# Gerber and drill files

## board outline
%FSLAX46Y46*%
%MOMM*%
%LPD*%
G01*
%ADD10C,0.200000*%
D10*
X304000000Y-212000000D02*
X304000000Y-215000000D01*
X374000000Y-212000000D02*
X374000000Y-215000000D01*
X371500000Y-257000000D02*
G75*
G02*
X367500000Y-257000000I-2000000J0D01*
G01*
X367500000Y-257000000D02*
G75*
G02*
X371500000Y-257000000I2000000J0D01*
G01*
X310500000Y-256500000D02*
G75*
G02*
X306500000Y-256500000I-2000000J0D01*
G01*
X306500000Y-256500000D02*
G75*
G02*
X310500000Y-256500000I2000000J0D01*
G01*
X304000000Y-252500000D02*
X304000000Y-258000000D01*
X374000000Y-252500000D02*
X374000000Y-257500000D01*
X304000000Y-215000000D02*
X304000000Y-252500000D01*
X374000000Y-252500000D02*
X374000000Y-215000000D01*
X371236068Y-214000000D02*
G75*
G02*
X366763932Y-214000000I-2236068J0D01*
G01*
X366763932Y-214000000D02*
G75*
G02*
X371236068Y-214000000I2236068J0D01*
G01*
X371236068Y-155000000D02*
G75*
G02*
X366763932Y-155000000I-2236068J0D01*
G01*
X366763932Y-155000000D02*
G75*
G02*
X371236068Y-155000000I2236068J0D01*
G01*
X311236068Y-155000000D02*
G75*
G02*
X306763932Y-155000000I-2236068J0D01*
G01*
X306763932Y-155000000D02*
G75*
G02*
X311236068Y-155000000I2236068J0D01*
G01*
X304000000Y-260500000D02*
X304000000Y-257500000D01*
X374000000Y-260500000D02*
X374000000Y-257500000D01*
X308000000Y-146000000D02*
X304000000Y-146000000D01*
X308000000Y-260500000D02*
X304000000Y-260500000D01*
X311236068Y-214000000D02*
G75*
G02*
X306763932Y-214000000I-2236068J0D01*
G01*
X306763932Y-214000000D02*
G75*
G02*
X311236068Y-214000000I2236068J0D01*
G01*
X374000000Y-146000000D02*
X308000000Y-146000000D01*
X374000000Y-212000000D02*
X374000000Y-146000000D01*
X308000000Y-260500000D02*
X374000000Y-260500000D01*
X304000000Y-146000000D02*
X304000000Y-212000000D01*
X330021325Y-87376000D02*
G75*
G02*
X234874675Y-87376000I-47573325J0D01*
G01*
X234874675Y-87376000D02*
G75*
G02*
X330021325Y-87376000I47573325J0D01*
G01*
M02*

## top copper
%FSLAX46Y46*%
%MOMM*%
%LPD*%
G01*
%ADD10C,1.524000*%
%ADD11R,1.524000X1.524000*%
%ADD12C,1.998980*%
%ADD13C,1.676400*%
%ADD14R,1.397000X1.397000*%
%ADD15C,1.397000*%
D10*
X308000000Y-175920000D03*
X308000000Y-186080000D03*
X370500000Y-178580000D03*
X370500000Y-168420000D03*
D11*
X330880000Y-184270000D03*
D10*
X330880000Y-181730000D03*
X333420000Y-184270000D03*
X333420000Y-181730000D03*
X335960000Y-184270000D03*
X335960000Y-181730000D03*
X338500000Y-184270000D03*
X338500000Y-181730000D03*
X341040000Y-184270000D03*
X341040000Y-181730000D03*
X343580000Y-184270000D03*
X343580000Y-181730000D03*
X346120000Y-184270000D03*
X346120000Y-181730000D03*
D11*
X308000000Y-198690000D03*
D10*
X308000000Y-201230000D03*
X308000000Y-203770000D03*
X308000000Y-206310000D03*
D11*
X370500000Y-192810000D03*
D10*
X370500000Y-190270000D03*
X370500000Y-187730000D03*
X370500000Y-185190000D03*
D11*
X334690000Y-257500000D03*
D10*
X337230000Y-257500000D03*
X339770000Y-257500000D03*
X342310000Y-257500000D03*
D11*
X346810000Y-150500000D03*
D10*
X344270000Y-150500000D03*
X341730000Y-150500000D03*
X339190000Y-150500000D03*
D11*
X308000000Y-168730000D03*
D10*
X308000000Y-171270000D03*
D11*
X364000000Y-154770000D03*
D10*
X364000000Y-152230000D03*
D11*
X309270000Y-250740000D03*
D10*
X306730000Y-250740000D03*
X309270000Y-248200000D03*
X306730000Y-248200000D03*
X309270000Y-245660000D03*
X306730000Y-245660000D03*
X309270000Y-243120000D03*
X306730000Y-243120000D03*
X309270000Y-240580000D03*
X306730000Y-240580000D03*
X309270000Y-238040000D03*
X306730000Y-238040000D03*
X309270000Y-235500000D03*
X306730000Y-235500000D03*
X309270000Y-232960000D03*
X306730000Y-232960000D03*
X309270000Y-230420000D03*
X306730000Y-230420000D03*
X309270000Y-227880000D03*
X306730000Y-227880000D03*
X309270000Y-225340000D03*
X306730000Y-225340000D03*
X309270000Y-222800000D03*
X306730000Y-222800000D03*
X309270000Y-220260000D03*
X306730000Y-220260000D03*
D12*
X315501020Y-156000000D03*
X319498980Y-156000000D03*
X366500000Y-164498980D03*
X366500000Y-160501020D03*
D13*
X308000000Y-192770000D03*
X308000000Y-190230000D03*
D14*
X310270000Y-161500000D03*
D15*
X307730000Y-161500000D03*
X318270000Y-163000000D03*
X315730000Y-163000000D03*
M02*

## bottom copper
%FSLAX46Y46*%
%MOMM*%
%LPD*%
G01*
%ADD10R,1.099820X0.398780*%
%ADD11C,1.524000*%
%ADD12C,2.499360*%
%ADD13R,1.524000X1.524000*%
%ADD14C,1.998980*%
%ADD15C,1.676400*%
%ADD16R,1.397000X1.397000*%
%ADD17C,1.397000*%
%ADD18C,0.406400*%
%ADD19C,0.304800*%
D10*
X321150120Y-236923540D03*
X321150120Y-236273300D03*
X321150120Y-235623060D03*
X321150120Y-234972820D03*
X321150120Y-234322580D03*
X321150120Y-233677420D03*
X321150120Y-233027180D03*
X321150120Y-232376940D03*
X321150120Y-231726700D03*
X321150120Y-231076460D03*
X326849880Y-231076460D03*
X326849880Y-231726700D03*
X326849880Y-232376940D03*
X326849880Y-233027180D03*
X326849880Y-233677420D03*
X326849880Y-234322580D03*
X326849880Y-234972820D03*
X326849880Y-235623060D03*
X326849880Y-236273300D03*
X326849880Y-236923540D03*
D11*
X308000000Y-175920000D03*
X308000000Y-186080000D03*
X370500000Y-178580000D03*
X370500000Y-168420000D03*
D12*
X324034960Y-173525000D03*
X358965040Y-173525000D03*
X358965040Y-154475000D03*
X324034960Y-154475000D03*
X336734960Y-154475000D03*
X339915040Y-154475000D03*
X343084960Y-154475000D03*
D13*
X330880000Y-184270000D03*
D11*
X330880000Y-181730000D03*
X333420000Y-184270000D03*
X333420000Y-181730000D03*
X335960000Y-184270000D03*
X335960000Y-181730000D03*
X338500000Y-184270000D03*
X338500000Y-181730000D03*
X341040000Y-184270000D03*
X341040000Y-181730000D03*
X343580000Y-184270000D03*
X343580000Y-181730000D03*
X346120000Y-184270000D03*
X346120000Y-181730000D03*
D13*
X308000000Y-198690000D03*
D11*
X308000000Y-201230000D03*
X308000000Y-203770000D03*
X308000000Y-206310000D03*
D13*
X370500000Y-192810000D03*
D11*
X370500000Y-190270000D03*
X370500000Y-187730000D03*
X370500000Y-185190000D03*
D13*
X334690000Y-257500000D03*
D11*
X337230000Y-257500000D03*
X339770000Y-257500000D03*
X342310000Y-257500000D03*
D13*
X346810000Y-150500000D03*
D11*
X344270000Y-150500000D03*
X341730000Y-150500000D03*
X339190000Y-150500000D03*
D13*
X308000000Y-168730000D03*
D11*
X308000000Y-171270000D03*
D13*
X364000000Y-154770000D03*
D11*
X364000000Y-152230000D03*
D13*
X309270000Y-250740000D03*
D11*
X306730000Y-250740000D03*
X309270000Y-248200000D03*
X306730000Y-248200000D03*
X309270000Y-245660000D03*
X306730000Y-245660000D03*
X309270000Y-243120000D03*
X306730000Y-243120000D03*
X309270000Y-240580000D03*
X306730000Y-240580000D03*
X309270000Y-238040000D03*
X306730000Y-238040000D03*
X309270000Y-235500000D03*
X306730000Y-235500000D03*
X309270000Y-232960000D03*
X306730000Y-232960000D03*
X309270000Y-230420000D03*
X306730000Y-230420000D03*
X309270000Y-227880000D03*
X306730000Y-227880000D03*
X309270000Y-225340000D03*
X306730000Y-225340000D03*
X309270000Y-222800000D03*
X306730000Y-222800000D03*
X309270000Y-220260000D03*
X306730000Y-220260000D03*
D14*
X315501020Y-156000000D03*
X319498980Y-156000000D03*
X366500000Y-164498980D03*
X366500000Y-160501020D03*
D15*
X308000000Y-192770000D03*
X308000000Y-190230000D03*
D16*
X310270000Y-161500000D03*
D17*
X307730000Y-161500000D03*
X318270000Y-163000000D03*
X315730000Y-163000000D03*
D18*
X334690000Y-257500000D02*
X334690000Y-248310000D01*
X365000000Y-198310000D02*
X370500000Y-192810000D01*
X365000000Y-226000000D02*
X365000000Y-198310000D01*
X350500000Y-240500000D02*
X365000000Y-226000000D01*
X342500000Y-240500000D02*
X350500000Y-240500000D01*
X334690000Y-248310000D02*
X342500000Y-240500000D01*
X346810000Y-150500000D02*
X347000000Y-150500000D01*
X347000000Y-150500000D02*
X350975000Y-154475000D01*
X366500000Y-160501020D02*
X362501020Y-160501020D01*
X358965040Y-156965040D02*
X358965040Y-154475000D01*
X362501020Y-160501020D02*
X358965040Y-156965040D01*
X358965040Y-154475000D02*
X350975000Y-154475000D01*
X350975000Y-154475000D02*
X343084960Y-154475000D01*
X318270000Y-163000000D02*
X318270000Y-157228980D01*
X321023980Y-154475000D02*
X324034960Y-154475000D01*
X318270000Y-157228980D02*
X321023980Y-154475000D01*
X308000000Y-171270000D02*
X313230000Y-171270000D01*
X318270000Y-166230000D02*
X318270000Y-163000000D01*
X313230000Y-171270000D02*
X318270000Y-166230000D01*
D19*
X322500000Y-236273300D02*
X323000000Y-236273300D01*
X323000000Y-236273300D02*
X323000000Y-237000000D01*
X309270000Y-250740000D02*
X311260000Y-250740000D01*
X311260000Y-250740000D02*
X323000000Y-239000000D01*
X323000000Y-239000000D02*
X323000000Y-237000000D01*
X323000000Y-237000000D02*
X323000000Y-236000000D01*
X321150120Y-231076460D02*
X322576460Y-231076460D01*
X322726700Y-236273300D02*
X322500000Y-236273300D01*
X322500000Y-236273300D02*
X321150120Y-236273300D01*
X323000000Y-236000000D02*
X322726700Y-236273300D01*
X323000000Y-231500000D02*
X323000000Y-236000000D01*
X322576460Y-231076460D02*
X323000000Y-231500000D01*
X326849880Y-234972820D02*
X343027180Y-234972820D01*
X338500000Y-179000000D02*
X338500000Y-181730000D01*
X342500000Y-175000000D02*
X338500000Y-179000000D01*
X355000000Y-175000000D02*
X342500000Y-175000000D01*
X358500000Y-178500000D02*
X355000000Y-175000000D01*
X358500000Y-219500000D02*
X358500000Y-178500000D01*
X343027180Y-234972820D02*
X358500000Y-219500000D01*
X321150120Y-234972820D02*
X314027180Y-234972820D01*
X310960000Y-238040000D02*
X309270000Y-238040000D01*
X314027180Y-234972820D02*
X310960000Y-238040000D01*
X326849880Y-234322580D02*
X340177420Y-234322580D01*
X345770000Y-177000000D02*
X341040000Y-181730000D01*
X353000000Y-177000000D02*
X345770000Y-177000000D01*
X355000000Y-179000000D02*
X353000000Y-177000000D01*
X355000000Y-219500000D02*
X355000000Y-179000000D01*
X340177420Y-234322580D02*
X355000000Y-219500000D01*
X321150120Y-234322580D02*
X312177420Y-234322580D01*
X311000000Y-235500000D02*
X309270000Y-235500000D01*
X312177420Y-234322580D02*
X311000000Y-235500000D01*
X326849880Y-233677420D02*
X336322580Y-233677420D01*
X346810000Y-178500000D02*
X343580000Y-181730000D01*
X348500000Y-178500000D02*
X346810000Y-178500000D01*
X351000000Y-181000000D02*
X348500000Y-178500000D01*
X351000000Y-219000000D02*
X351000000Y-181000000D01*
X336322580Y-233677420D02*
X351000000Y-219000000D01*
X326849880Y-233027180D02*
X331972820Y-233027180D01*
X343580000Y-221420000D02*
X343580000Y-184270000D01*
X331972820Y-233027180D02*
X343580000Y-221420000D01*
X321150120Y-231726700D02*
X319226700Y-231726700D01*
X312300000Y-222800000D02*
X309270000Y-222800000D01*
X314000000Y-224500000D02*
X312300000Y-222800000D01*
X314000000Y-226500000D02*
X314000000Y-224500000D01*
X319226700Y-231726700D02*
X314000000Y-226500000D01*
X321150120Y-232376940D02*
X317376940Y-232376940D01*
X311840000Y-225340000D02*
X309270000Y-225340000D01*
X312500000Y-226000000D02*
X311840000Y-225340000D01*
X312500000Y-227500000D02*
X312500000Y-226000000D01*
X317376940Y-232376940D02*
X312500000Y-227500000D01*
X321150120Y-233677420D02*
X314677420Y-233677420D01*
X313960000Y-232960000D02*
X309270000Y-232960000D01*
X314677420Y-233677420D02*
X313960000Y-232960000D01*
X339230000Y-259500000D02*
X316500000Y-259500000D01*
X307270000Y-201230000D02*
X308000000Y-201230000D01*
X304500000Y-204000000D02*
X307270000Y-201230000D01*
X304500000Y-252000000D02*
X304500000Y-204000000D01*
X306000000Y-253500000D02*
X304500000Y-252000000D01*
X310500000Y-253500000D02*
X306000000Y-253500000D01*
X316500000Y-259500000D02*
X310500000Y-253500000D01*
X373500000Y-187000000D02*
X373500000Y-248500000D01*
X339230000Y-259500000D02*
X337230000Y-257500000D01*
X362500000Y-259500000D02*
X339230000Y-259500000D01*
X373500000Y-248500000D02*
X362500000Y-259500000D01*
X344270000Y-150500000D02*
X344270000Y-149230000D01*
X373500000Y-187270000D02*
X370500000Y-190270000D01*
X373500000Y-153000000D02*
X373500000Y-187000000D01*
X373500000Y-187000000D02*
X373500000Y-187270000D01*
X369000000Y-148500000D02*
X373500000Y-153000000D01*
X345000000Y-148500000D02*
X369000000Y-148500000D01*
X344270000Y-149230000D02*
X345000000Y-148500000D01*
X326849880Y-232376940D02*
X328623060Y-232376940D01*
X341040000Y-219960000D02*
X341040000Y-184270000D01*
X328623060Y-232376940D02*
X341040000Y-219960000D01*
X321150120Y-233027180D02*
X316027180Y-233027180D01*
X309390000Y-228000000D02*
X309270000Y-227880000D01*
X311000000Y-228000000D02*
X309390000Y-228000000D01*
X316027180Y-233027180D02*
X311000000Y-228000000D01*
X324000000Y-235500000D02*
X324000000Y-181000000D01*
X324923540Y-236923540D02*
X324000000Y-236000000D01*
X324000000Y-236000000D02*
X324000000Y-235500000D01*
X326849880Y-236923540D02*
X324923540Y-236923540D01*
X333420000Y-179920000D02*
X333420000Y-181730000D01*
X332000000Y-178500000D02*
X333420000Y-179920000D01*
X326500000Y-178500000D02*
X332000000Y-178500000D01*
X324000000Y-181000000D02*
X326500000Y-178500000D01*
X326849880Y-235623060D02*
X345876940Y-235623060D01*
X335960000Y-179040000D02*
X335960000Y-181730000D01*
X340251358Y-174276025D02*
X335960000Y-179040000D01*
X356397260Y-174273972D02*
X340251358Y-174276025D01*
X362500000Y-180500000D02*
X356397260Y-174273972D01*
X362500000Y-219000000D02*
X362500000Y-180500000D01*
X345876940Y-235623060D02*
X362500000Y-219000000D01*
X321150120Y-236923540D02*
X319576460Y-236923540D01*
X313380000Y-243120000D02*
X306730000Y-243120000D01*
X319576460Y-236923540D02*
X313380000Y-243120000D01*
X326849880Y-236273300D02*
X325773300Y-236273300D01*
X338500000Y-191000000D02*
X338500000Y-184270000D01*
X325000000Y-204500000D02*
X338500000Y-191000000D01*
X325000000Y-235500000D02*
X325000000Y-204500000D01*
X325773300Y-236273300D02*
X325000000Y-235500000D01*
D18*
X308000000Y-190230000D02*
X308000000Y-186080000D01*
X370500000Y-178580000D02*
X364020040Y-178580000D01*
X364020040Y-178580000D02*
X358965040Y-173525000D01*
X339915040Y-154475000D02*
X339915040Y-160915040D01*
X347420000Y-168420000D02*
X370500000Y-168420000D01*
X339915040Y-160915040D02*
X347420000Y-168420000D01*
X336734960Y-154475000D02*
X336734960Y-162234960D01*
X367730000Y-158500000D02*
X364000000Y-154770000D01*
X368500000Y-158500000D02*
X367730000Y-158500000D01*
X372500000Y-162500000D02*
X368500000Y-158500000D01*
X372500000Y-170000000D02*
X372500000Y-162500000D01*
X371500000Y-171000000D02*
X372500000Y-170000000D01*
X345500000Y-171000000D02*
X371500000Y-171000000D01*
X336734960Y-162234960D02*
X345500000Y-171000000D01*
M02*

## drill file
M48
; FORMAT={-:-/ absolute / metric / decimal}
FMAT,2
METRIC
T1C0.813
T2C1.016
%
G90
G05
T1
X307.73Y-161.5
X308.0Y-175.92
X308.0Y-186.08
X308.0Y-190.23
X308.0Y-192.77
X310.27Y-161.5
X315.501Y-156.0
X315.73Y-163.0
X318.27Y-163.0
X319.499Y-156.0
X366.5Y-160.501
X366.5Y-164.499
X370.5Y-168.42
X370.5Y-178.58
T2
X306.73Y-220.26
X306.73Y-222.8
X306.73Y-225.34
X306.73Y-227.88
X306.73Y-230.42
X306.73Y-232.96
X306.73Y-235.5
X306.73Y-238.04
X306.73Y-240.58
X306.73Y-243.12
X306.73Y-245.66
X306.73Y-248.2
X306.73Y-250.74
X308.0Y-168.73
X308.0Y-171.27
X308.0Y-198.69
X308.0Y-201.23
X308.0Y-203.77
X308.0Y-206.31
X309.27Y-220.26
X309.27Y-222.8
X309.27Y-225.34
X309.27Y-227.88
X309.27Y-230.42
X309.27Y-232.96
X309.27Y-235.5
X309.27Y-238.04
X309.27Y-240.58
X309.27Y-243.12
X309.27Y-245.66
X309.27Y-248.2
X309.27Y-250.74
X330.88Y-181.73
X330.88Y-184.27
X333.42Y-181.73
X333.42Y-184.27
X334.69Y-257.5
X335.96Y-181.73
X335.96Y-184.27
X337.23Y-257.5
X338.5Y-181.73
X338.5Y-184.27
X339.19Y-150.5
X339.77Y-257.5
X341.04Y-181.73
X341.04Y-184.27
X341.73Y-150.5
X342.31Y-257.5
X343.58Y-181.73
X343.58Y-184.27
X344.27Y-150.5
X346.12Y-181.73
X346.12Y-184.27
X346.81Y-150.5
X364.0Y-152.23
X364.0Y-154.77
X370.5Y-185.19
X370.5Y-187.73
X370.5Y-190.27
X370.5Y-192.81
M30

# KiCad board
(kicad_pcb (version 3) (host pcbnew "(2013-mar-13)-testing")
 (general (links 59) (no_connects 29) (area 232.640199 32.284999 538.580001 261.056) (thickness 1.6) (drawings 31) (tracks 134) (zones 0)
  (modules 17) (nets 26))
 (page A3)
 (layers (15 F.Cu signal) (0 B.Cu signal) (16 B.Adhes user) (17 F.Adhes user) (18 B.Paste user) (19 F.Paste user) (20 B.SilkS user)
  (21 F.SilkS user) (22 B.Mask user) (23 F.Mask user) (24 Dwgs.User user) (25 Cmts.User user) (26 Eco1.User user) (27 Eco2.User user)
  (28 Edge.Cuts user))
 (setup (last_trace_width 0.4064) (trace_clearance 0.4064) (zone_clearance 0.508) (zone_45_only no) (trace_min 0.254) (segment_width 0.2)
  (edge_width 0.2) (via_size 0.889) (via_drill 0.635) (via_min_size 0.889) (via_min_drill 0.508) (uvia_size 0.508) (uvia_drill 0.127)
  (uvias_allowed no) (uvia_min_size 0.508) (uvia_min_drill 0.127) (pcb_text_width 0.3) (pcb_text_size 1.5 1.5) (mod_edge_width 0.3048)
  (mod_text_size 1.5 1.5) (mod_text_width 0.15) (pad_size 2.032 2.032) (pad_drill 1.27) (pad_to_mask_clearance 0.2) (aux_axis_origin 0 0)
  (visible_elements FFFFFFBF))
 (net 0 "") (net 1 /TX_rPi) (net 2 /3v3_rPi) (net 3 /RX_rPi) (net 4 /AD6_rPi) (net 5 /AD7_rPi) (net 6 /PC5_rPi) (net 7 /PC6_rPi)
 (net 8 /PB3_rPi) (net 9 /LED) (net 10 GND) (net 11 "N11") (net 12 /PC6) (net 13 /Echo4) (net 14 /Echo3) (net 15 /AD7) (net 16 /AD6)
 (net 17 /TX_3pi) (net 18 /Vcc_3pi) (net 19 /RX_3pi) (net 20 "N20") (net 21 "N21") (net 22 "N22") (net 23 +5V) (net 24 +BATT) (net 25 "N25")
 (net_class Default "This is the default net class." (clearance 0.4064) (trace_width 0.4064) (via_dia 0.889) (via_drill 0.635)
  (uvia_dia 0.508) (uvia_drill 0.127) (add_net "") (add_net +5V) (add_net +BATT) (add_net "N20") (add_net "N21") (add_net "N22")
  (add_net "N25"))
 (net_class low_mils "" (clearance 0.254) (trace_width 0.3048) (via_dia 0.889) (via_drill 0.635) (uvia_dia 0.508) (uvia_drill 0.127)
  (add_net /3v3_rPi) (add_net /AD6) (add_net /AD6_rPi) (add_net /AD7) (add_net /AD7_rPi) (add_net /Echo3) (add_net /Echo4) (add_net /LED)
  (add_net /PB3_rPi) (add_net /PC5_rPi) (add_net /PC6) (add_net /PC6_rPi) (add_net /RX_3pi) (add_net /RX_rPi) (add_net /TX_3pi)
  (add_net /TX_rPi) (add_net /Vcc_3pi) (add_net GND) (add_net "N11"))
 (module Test (layer B.Cu) (at 324 234 90)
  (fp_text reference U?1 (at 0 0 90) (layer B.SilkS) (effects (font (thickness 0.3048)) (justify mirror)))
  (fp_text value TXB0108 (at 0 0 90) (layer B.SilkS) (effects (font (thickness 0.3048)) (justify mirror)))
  (pad 1 smd rect (at -2.92354 -2.84988 270) (size 0.39878 1.09982) (layers B.Cu B.Paste B.Mask) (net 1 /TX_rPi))
  (pad 2 smd rect (at -2.2733 -2.84988 270) (size 0.39878 1.09982) (layers B.Cu B.Paste B.Mask) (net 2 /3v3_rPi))
  (pad 3 smd rect (at -1.62306 -2.84988 270) (size 0.39878 1.09982) (layers B.Cu B.Paste B.Mask) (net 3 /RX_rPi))
  (pad 4 smd rect (at -0.97282 -2.84988 270) (size 0.39878 1.09982) (layers B.Cu B.Paste B.Mask) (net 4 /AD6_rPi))
  (pad 5 smd rect (at -0.32258 -2.84988 270) (size 0.39878 1.09982) (layers B.Cu B.Paste B.Mask) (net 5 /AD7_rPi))
  (pad 6 smd rect (at 0.32258 -2.84988 270) (size 0.39878 1.09982) (layers B.Cu B.Paste B.Mask) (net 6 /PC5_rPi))
  (pad 7 smd rect (at 0.97282 -2.84988 270) (size 0.39878 1.09982) (layers B.Cu B.Paste B.Mask) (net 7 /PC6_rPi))
  (pad 8 smd rect (at 1.62306 -2.84988 270) (size 0.39878 1.09982) (layers B.Cu B.Paste B.Mask) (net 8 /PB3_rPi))
  (pad 9 smd rect (at 2.2733 -2.84988 270) (size 0.39878 1.09982) (layers B.Cu B.Paste B.Mask) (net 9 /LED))
  (pad 10 smd rect (at 2.92354 -2.84988 270) (size 0.39878 1.09982) (layers B.Cu B.Paste B.Mask) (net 2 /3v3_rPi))
  (pad 11 smd rect (at 2.92354 2.84988 90) (size 0.39878 1.09982) (layers B.Cu B.Paste B.Mask) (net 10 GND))
  (pad 12 smd rect (at 2.2733 2.84988 90) (size 0.39878 1.09982) (layers B.Cu B.Paste B.Mask) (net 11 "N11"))
  (pad 13 smd rect (at 1.62306 2.84988 90) (size 0.39878 1.09982) (layers B.Cu B.Paste B.Mask) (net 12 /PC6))
  (pad 14 smd rect (at 0.97282 2.84988 90) (size 0.39878 1.09982) (layers B.Cu B.Paste B.Mask) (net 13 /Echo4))
  (pad 15 smd rect (at 0.32258 2.84988 90) (size 0.39878 1.09982) (layers B.Cu B.Paste B.Mask) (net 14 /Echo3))
  (pad 16 smd rect (at -0.32258 2.84988 90) (size 0.39878 1.09982) (layers B.Cu B.Paste B.Mask) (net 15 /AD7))
  (pad 17 smd rect (at -0.97282 2.84988 90) (size 0.39878 1.09982) (layers B.Cu B.Paste B.Mask) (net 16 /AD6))
  (pad 18 smd rect (at -1.62306 2.84988 90) (size 0.39878 1.09982) (layers B.Cu B.Paste B.Mask) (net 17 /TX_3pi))
  (pad 19 smd rect (at -2.2733 2.84988 90) (size 0.39878 1.09982) (layers B.Cu B.Paste B.Mask) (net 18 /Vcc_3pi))
  (pad 20 smd rect (at -2.92354 2.84988 90) (size 0.39878 1.09982) (layers B.Cu B.Paste B.Mask) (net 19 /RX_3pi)))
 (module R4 (layer F.Cu) (at 308 181 270) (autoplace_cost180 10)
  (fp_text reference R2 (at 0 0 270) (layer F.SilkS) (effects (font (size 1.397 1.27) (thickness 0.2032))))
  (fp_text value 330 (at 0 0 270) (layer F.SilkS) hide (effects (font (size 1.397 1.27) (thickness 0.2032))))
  (pad 1 thru_hole circle (at -5.08 0 270) (size 1.524 1.524) (drill 0.8128) (layers *.Cu *.Mask F.SilkS) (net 10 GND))
  (pad 2 thru_hole circle (at 5.08 0 270) (size 1.524 1.524) (drill 0.8128) (layers *.Cu *.Mask F.SilkS) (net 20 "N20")))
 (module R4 (layer F.Cu) (at 370.5 173.5 90) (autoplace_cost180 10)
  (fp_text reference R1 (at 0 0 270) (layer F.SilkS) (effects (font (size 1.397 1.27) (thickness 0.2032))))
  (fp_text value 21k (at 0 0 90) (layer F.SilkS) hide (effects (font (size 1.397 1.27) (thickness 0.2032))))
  (pad 1 thru_hole circle (at -5.08 0 90) (size 1.524 1.524) (drill 0.8128) (layers *.Cu *.Mask F.SilkS) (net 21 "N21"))
  (pad 2 thru_hole circle (at 5.08 0 90) (size 1.524 1.524) (drill 0.8128) (layers *.Cu *.Mask F.SilkS) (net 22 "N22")))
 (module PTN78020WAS (layer B.Cu) (at 341.5 164)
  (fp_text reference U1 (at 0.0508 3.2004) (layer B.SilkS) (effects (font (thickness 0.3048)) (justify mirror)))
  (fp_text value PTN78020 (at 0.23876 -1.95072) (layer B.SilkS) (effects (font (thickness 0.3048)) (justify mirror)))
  (pad 1 smd circle (at -17.46504 9.525) (size 2.49936 2.49936) (layers B.Cu B.Paste B.Mask) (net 10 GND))
  (pad 7 smd circle (at 17.46504 9.525) (size 2.49936 2.49936) (layers B.Cu B.Paste B.Mask) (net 21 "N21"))
  (pad 6 smd circle (at 17.46504 -9.525) (size 2.49936 2.49936) (layers B.Cu B.Paste B.Mask) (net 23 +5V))
  (pad 2 smd circle (at -17.46504 -9.525) (size 2.49936 2.49936) (layers B.Cu B.Paste B.Mask) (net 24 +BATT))
  (pad 3 smd circle (at -4.76504 -9.525) (size 2.49936 2.49936) (layers B.Cu B.Paste B.Mask) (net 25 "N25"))
  (pad 4 smd circle (at -1.58496 -9.525) (size 2.49936 2.49936) (layers B.Cu B.Paste B.Mask) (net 22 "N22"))
  (pad 5 smd circle (at 1.58496 -9.525) (size 2.49936 2.49936) (layers B.Cu B.Paste B.Mask) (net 23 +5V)))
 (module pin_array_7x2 (layer F.Cu) (at 338.5 183)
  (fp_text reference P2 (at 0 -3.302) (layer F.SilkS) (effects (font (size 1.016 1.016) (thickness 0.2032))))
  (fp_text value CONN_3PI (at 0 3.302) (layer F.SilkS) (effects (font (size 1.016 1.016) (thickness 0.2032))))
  (pad 1 thru_hole rect (at -7.62 1.27) (size 1.524 1.524) (drill 1.016) (layers *.Cu *.Mask F.SilkS) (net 10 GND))
  (pad 2 thru_hole circle (at -7.62 -1.27) (size 1.524 1.524) (drill 1.016) (layers *.Cu *.Mask F.SilkS) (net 10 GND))
  (pad 3 thru_hole circle (at -5.08 1.27) (size 1.524 1.524) (drill 1.016) (layers *.Cu *.Mask F.SilkS))
  (pad 4 thru_hole circle (at -5.08 -1.27) (size 1.524 1.524) (drill 1.016) (layers *.Cu *.Mask F.SilkS) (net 19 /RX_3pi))
  (pad 5 thru_hole circle (at -2.54 1.27) (size 1.524 1.524) (drill 1.016) (layers *.Cu *.Mask F.SilkS))
  (pad 6 thru_hole circle (at -2.54 -1.27) (size 1.524 1.524) (drill 1.016) (layers *.Cu *.Mask F.SilkS) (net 17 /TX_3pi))
  (pad 7 thru_hole circle (at 0 1.27) (size 1.524 1.524) (drill 1.016) (layers *.Cu *.Mask F.SilkS) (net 18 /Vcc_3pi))
  (pad 8 thru_hole circle (at 0 -1.27) (size 1.524 1.524) (drill 1.016) (layers *.Cu *.Mask F.SilkS) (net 16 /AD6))
  (pad 9 thru_hole circle (at 2.54 1.27) (size 1.524 1.524) (drill 1.016) (layers *.Cu *.Mask F.SilkS) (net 12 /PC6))
  (pad 10 thru_hole circle (at 2.54 -1.27) (size 1.524 1.524) (drill 1.016) (layers *.Cu *.Mask F.SilkS) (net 15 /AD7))
  (pad 11 thru_hole circle (at 5.08 1.27) (size 1.524 1.524) (drill 1.016) (layers *.Cu *.Mask F.SilkS) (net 13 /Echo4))
  (pad 12 thru_hole circle (at 5.08 -1.27) (size 1.524 1.524) (drill 1.016) (layers *.Cu *.Mask F.SilkS) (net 14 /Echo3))
  (pad 13 thru_hole circle (at 7.62 1.27) (size 1.524 1.524) (drill 1.016) (layers *.Cu *.Mask F.SilkS) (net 10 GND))
  (pad 14 thru_hole circle (at 7.62 -1.27) (size 1.524 1.524) (drill 1.016) (layers *.Cu *.Mask F.SilkS) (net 10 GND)))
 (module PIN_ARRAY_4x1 (layer F.Cu) (at 308 202.5 270)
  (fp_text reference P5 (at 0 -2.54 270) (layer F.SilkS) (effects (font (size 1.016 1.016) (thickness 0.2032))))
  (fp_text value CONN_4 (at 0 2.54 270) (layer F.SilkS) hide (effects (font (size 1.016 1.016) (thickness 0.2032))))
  (pad 1 thru_hole rect (at -3.81 0 270) (size 1.524 1.524) (drill 1.016) (layers *.Cu *.Mask F.SilkS) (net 23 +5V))
  (pad 2 thru_hole circle (at -1.27 0 270) (size 1.524 1.524) (drill 1.016) (layers *.Cu *.Mask F.SilkS) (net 12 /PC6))
  (pad 3 thru_hole circle (at 1.27 0 270) (size 1.524 1.524) (drill 1.016) (layers *.Cu *.Mask F.SilkS) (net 16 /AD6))
  (pad 4 thru_hole circle (at 3.81 0 270) (size 1.524 1.524) (drill 1.016) (layers *.Cu *.Mask F.SilkS) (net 10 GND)))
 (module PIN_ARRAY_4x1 (layer F.Cu) (at 370.5 189 90)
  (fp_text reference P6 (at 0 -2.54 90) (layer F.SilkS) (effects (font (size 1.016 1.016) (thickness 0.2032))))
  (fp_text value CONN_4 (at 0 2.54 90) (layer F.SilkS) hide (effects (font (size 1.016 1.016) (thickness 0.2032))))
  (pad 1 thru_hole rect (at -3.81 0 90) (size 1.524 1.524) (drill 1.016) (layers *.Cu *.Mask F.SilkS) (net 23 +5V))
  (pad 2 thru_hole circle (at -1.27 0 90) (size 1.524 1.524) (drill 1.016) (layers *.Cu *.Mask F.SilkS) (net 12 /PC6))
  (pad 3 thru_hole circle (at 1.27 0 90) (size 1.524 1.524) (drill 1.016) (layers *.Cu *.Mask F.SilkS) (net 15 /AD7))
  (pad 4 thru_hole circle (at 3.81 0 90) (size 1.524 1.524) (drill 1.016) (layers *.Cu *.Mask F.SilkS) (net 10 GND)))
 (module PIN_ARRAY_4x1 (layer F.Cu) (at 338.5 257.5)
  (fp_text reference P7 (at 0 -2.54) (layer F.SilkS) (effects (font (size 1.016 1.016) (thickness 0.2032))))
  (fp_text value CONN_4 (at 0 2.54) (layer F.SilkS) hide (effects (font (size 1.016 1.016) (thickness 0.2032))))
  (pad 1 thru_hole rect (at -3.81 0) (size 1.524 1.524) (drill 1.016) (layers *.Cu *.Mask F.SilkS) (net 23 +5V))
  (pad 2 thru_hole circle (at -1.27 0) (size 1.524 1.524) (drill 1.016) (layers *.Cu *.Mask F.SilkS) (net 12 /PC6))
  (pad 3 thru_hole circle (at 1.27 0) (size 1.524 1.524) (drill 1.016) (layers *.Cu *.Mask F.SilkS) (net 14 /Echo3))
  (pad 4 thru_hole circle (at 3.81 0) (size 1.524 1.524) (drill 1.016) (layers *.Cu *.Mask F.SilkS) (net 10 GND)))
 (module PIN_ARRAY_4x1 (layer F.Cu) (at 343 150.5 180)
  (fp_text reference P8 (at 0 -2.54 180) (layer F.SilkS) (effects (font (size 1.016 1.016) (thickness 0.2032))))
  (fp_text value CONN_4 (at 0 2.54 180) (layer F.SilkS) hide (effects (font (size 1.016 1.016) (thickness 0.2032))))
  (pad 1 thru_hole rect (at -3.81 0 180) (size 1.524 1.524) (drill 1.016) (layers *.Cu *.Mask F.SilkS) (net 23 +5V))
  (pad 2 thru_hole circle (at -1.27 0 180) (size 1.524 1.524) (drill 1.016) (layers *.Cu *.Mask F.SilkS) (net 12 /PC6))
  (pad 3 thru_hole circle (at 1.27 0 180) (size 1.524 1.524) (drill 1.016) (layers *.Cu *.Mask F.SilkS) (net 13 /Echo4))
  (pad 4 thru_hole circle (at 3.81 0 180) (size 1.524 1.524) (drill 1.016) (layers *.Cu *.Mask F.SilkS) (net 10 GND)))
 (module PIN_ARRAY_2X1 (layer F.Cu) (at 308 170 270)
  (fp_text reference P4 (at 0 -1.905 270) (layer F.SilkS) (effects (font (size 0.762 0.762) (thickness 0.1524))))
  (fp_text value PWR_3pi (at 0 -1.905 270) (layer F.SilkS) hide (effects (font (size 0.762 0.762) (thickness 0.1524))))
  (pad 1 thru_hole rect (at -1.27 0 270) (size 1.524 1.524) (drill 1.016) (layers *.Cu *.Mask F.SilkS) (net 10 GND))
  (pad 2 thru_hole circle (at 1.27 0 270) (size 1.524 1.524) (drill 1.016) (layers *.Cu *.Mask F.SilkS) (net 24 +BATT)))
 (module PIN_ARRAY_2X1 (layer F.Cu) (at 364 153.5 90)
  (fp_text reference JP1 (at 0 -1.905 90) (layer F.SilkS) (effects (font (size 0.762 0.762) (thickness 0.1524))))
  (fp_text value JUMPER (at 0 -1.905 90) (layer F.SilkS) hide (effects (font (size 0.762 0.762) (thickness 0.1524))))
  (pad 1 thru_hole rect (at -1.27 0 90) (size 1.524 1.524) (drill 1.016) (layers *.Cu *.Mask F.SilkS) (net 25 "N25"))
  (pad 2 thru_hole circle (at 1.27 0 90) (size 1.524 1.524) (drill 1.016) (layers *.Cu *.Mask F.SilkS) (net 10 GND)))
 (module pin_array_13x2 (layer F.Cu) (at 308 235.5 90)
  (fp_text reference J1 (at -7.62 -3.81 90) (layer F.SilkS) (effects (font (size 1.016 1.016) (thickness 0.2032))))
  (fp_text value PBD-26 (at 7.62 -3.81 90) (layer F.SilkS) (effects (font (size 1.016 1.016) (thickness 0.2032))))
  (pad 1 thru_hole rect (at -15.24 1.27 90) (size 1.524 1.524) (drill 1.016) (layers *.Cu *.Mask F.SilkS) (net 2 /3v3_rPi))
  (pad 2 thru_hole circle (at -15.24 -1.27 90) (size 1.524 1.524) (drill 1.016) (layers *.Cu *.Mask F.SilkS))
  (pad 3 thru_hole circle (at -12.7 1.27 90) (size 1.524 1.524) (drill 1.016) (layers *.Cu *.Mask F.SilkS))
  (pad 4 thru_hole circle (at -12.7 -1.27 90) (size 1.524 1.524) (drill 1.016) (layers *.Cu *.Mask F.SilkS))
  (pad 5 thru_hole circle (at -10.16 1.27 90) (size 1.524 1.524) (drill 1.016) (layers *.Cu *.Mask F.SilkS))
  (pad 6 thru_hole circle (at -10.16 -1.27 90) (size 1.524 1.524) (drill 1.016) (layers *.Cu *.Mask F.SilkS) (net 10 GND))
  (pad 7 thru_hole circle (at -7.62 1.27 90) (size 1.524 1.524) (drill 1.016) (layers *.Cu *.Mask F.SilkS) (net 1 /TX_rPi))
  (pad 8 thru_hole circle (at -7.62 -1.27 90) (size 1.524 1.524) (drill 1.016) (layers *.Cu *.Mask F.SilkS) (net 1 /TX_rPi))
  (pad 9 thru_hole circle (at -5.08 1.27 90) (size 1.524 1.524) (drill 1.016) (layers *.Cu *.Mask F.SilkS))
  (pad 10 thru_hole circle (at -5.08 -1.27 90) (size 1.524 1.524) (drill 1.016) (layers *.Cu *.Mask F.SilkS) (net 3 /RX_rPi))
  (pad 11 thru_hole circle (at -2.54 1.27 90) (size 1.524 1.524) (drill 1.016) (layers *.Cu *.Mask F.SilkS) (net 4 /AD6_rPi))
  (pad 12 thru_hole circle (at -2.54 -1.27 90) (size 1.524 1.524) (drill 1.016) (layers *.Cu *.Mask F.SilkS))
  (pad 13 thru_hole circle (at 0 1.27 90) (size 1.524 1.524) (drill 1.016) (layers *.Cu *.Mask F.SilkS) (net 5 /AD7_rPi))
  (pad 14 thru_hole circle (at 0 -1.27 90) (size 1.524 1.524) (drill 1.016) (layers *.Cu *.Mask F.SilkS))
  (pad 15 thru_hole circle (at 2.54 1.27 90) (size 1.524 1.524) (drill 1.016) (layers *.Cu *.Mask F.SilkS) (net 6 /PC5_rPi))
  (pad 16 thru_hole circle (at 2.54 -1.27 90) (size 1.524 1.524) (drill 1.016) (layers *.Cu *.Mask F.SilkS))
  (pad 17 thru_hole circle (at 5.08 1.27 90) (size 1.524 1.524) (drill 1.016) (layers *.Cu *.Mask F.SilkS))
  (pad 18 thru_hole circle (at 5.08 -1.27 90) (size 1.524 1.524) (drill 1.016) (layers *.Cu *.Mask F.SilkS))
  (pad 19 thru_hole circle (at 7.62 1.27 90) (size 1.524 1.524) (drill 1.016) (layers *.Cu *.Mask F.SilkS) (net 7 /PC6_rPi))
  (pad 20 thru_hole circle (at 7.62 -1.27 90) (size 1.524 1.524) (drill 1.016) (layers *.Cu *.Mask F.SilkS))
  (pad 21 thru_hole circle (at 10.16 1.27 90) (size 1.524 1.524) (drill 1.016) (layers *.Cu *.Mask F.SilkS) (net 8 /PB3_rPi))
  (pad 22 thru_hole circle (at 10.16 -1.27 90) (size 1.524 1.524) (drill 1.016) (layers *.Cu *.Mask F.SilkS))
  (pad 23 thru_hole circle (at 12.7 1.27 90) (size 1.524 1.524) (drill 1.016) (layers *.Cu *.Mask F.SilkS) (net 9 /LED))
  (pad 24 thru_hole circle (at 12.7 -1.27 90) (size 1.524 1.524) (drill 1.016) (layers *.Cu *.Mask F.SilkS))
  (pad 25 thru_hole circle (at 15.24 1.27 90) (size 1.524 1.524) (drill 1.016) (layers *.Cu *.Mask F.SilkS))
  (pad 26 thru_hole circle (at 15.24 -1.27 90) (size 1.524 1.524) (drill 1.016) (layers *.Cu *.Mask F.SilkS)))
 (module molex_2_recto (layer F.Cu) (at 317.5 156 180)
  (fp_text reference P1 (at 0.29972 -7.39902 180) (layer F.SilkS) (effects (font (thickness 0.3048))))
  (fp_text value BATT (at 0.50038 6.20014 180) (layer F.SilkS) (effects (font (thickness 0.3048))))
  (pad 1 thru_hole circle (at 1.99898 0 180) (size 1.99898 1.99898) (drill 0.8128) (layers *.Cu *.Mask F.SilkS) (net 10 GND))
  (pad 2 thru_hole circle (at -1.99898 0 180) (size 1.99898 1.99898) (drill 0.8128) (layers *.Cu *.Mask F.SilkS) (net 24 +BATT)))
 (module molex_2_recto (layer F.Cu) (at 366.5 162.5 270)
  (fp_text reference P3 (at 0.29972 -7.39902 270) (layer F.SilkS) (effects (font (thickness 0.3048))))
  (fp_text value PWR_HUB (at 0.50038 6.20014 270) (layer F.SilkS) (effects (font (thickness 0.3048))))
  (pad 1 thru_hole circle (at 1.99898 0 270) (size 1.99898 1.99898) (drill 0.8128) (layers *.Cu *.Mask F.SilkS) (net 10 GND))
  (pad 2 thru_hole circle (at -1.99898 0 270) (size 1.99898 1.99898) (drill 0.8128) (layers *.Cu *.Mask F.SilkS) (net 23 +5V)))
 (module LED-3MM (layer F.Cu) (at 308 191.5 90)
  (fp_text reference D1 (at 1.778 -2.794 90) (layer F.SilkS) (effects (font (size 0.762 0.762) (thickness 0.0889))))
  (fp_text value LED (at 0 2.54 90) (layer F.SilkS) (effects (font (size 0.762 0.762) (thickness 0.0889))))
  (pad 1 thru_hole circle (at -1.27 0 90) (size 1.6764 1.6764) (drill 0.8128) (layers *.Cu *.Mask F.SilkS) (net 11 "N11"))
  (pad 2 thru_hole circle (at 1.27 0 90) (size 1.6764 1.6764) (drill 0.8128) (layers *.Cu *.Mask F.SilkS) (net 20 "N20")))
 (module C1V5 (layer F.Cu) (at 309 161.5 180)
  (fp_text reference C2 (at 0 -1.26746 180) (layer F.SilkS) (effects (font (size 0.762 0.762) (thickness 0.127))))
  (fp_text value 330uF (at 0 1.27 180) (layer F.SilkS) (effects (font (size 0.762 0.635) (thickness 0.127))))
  (pad 1 thru_hole rect (at -1.27 0 180) (size 1.397 1.397) (drill 0.8128) (layers *.Cu *.Mask F.SilkS) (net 23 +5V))
  (pad 2 thru_hole circle (at 1.27 0 180) (size 1.397 1.397) (drill 0.8128) (layers *.Cu *.Mask F.SilkS) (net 10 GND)))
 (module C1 (layer F.Cu) (at 317 163 180)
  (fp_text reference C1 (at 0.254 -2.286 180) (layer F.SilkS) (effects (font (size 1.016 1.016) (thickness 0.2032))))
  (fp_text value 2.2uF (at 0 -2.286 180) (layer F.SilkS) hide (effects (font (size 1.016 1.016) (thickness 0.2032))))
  (pad 1 thru_hole circle (at -1.27 0 180) (size 1.397 1.397) (drill 0.8128) (layers *.Cu *.Mask F.SilkS) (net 24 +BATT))
  (pad 2 thru_hole circle (at 1.27 0 180) (size 1.397 1.397) (drill 0.8128) (layers *.Cu *.Mask F.SilkS) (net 10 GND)))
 (gr_line (start 304 212) (end 304 215) (angle 90) (layer Edge.Cuts) (width 0.2))
 (gr_line (start 374 212) (end 374 215) (angle 90) (layer Edge.Cuts) (width 0.2))
 (gr_circle (center 369.5 257) (end 369.5 259) (layer Edge.Cuts) (width 0.2))
 (gr_circle (center 308.5 256.5) (end 308.5 258.5) (layer Edge.Cuts) (width 0.2))
 (gr_line (start 304 252.5) (end 304 258) (angle 90) (layer Edge.Cuts) (width 0.2))
 (gr_line (start 374 252.5) (end 374 257.5) (angle 90) (layer Edge.Cuts) (width 0.2))
 (gr_line (start 304 215) (end 304 252.5) (angle 90) (layer Edge.Cuts) (width 0.2))
 (gr_line (start 374 252.5) (end 374 215) (angle 90) (layer Edge.Cuts) (width 0.2))
 (gr_circle (center 369 214) (end 370 216) (layer Edge.Cuts) (width 0.2))
 (gr_circle (center 369 155) (end 367 156) (layer Edge.Cuts) (width 0.2))
 (gr_circle (center 309 155) (end 311 156) (layer Edge.Cuts) (width 0.2))
 (gr_line (start 304 260.5) (end 304 257.5) (angle 90) (layer Edge.Cuts) (width 0.2))
 (gr_line (start 374 260.5) (end 374 257.5) (angle 90) (layer Edge.Cuts) (width 0.2))
 (gr_line (start 308 146) (end 304 146) (angle 90) (layer Edge.Cuts) (width 0.2))
 (gr_line (start 308 260.5) (end 304 260.5) (angle 90) (layer Edge.Cuts) (width 0.2))
 (gr_circle (center 309 214) (end 311 215) (layer Edge.Cuts) (width 0.2))
 (gr_line (start 374 146) (end 308 146) (angle 90) (layer Edge.Cuts) (width 0.2))
 (gr_line (start 374 212) (end 374 146) (angle 90) (layer Edge.Cuts) (width 0.2))
 (gr_line (start 308 260.5) (end 374 260.5) (angle 90) (layer Edge.Cuts) (width 0.2))
 (gr_line (start 304 146) (end 304 212) (angle 90) (layer Edge.Cuts) (width 0.2))
 (gr_circle (center 282.448 87.376) (end 329.692 92.964) (layer Edge.Cuts) (width 0.2))
 (segment (start 334.69 257.5) (end 334.69 248.31) (width 0.4064) (layer B.Cu) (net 23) (status 400000))
 (segment (start 365 198.31) (end 370.5 192.81) (width 0.4064) (layer B.Cu) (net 23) (status 800000))
 (segment (start 365 226) (end 365 198.31) (width 0.4064) (layer B.Cu) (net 23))
 (segment (start 350.5 240.5) (end 365 226) (width 0.4064) (layer B.Cu) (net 23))
 (segment (start 342.5 240.5) (end 350.5 240.5) (width 0.4064) (layer B.Cu) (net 23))
 (segment (start 334.69 248.31) (end 342.5 240.5) (width 0.4064) (layer B.Cu) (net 23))
 (segment (start 346.81 150.5) (end 347 150.5) (width 0.4064) (layer B.Cu) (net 23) (status C00000))
 (segment (start 347 150.5) (end 350.975 154.475) (width 0.4064) (layer B.Cu) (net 23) (status 400000))
 (segment (start 366.5 160.50102) (end 362.50102 160.50102) (width 0.4064) (layer B.Cu) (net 23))
 (segment (start 358.96504 156.96504) (end 358.96504 154.475) (width 0.4064) (layer B.Cu) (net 23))
 (segment (start 362.50102 160.50102) (end 358.96504 156.96504) (width 0.4064) (layer B.Cu) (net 23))
 (segment (start 358.96504 154.475) (end 350.975 154.475) (width 0.4064) (layer B.Cu) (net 23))
 (segment (start 350.975 154.475) (end 343.08496 154.475) (width 0.4064) (layer B.Cu) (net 23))
 (segment (start 318.27 163) (end 318.27 157.22898) (width 0.4064) (layer B.Cu) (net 24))
 (segment (start 321.02398 154.475) (end 324.03496 154.475) (width 0.4064) (layer B.Cu) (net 24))
 (segment (start 318.27 157.22898) (end 321.02398 154.475) (width 0.4064) (layer B.Cu) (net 24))
 (segment (start 308 171.27) (end 313.23 171.27) (width 0.4064) (layer B.Cu) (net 24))
 (segment (start 318.27 166.23) (end 318.27 163) (width 0.4064) (layer B.Cu) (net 24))
 (segment (start 313.23 171.27) (end 318.27 166.23) (width 0.4064) (layer B.Cu) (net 24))
 (segment (start 322.5 236.2733) (end 323 236.2733) (width 0.3048) (layer B.Cu) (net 2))
 (segment (start 323 236.2733) (end 323 237) (width 0.3048) (layer B.Cu) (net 2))
 (segment (start 309.27 250.74) (end 311.26 250.74) (width 0.3048) (layer B.Cu) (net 2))
 (segment (start 311.26 250.74) (end 323 239) (width 0.3048) (layer B.Cu) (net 2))
 (segment (start 323 239) (end 323 237) (width 0.3048) (layer B.Cu) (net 2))
 (segment (start 323 237) (end 323 236) (width 0.3048) (layer B.Cu) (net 2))
 (segment (start 321.15012 231.07646) (end 322.57646 231.07646) (width 0.3048) (layer B.Cu) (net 2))
 (segment (start 322.7267 236.2733) (end 322.5 236.2733) (width 0.3048) (layer B.Cu) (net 2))
 (segment (start 322.5 236.2733) (end 321.15012 236.2733) (width 0.3048) (layer B.Cu) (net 2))
 (segment (start 323 236) (end 322.7267 236.2733) (width 0.3048) (layer B.Cu) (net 2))
 (segment (start 323 231.5) (end 323 236) (width 0.3048) (layer B.Cu) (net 2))
 (segment (start 322.57646 231.07646) (end 323 231.5) (width 0.3048) (layer B.Cu) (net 2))
 (segment (start 326.84988 234.97282) (end 343.02718 234.97282) (width 0.3048) (layer B.Cu) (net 16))
 (segment (start 338.5 179) (end 338.5 181.73) (width 0.3048) (layer B.Cu) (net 16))
 (segment (start 342.5 175) (end 338.5 179) (width 0.3048) (layer B.Cu) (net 16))
 (segment (start 355 175) (end 342.5 175) (width 0.3048) (layer B.Cu) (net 16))
 (segment (start 358.5 178.5) (end 355 175) (width 0.3048) (layer B.Cu) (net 16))
 (segment (start 358.5 219.5) (end 358.5 178.5) (width 0.3048) (layer B.Cu) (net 16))
 (segment (start 343.02718 234.97282) (end 358.5 219.5) (width 0.3048) (layer B.Cu) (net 16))
 (segment (start 321.15012 234.97282) (end 314.02718 234.97282) (width 0.3048) (layer B.Cu) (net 4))
 (segment (start 310.96 238.04) (end 309.27 238.04) (width 0.3048) (layer B.Cu) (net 4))
 (segment (start 314.02718 234.97282) (end 310.96 238.04) (width 0.3048) (layer B.Cu) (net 4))
 (segment (start 326.84988 234.32258) (end 340.17742 234.32258) (width 0.3048) (layer B.Cu) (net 15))
 (segment (start 345.77 177) (end 341.04 181.73) (width 0.3048) (layer B.Cu) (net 15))
 (segment (start 353 177) (end 345.77 177) (width 0.3048) (layer B.Cu) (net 15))
 (segment (start 355 179) (end 353 177) (width 0.3048) (layer B.Cu) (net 15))
 (segment (start 355 219.5) (end 355 179) (width 0.3048) (layer B.Cu) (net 15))
 (segment (start 340.17742 234.32258) (end 355 219.5) (width 0.3048) (layer B.Cu) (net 15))
 (segment (start 321.15012 234.32258) (end 312.17742 234.32258) (width 0.3048) (layer B.Cu) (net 5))
 (segment (start 311 235.5) (end 309.27 235.5) (width 0.3048) (layer B.Cu) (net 5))
 (segment (start 312.17742 234.32258) (end 311 235.5) (width 0.3048) (layer B.Cu) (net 5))
 (segment (start 326.84988 233.67742) (end 336.32258 233.67742) (width 0.3048) (layer B.Cu) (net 14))
 (segment (start 346.81 178.5) (end 343.58 181.73) (width 0.3048) (layer B.Cu) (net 14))
 (segment (start 348.5 178.5) (end 346.81 178.5) (width 0.3048) (layer B.Cu) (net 14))
 (segment (start 351 181) (end 348.5 178.5) (width 0.3048) (layer B.Cu) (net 14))
 (segment (start 351 219) (end 351 181) (width 0.3048) (layer B.Cu) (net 14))
 (segment (start 336.32258 233.67742) (end 351 219) (width 0.3048) (layer B.Cu) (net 14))
 (segment (start 326.84988 233.02718) (end 331.97282 233.02718) (width 0.3048) (layer B.Cu) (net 13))
 (segment (start 343.58 221.42) (end 343.58 184.27) (width 0.3048) (layer B.Cu) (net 13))
 (segment (start 331.97282 233.02718) (end 343.58 221.42) (width 0.3048) (layer B.Cu) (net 13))
 (segment (start 321.15012 231.7267) (end 319.2267 231.7267) (width 0.3048) (layer B.Cu) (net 9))
 (segment (start 312.3 222.8) (end 309.27 222.8) (width 0.3048) (layer B.Cu) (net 9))
 (segment (start 314 224.5) (end 312.3 222.8) (width 0.3048) (layer B.Cu) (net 9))
 (segment (start 314 226.5) (end 314 224.5) (width 0.3048) (layer B.Cu) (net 9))
 (segment (start 319.2267 231.7267) (end 314 226.5) (width 0.3048) (layer B.Cu) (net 9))
 (segment (start 321.15012 232.37694) (end 317.37694 232.37694) (width 0.3048) (layer B.Cu) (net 8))
 (segment (start 311.84 225.34) (end 309.27 225.34) (width 0.3048) (layer B.Cu) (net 8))
 (segment (start 312.5 226) (end 311.84 225.34) (width 0.3048) (layer B.Cu) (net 8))
 (segment (start 312.5 227.5) (end 312.5 226) (width 0.3048) (layer B.Cu) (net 8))
 (segment (start 317.37694 232.37694) (end 312.5 227.5) (width 0.3048) (layer B.Cu) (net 8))
 (segment (start 321.15012 233.67742) (end 314.67742 233.67742) (width 0.3048) (layer B.Cu) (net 6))
 (segment (start 313.96 232.96) (end 309.27 232.96) (width 0.3048) (layer B.Cu) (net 6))
 (segment (start 314.67742 233.67742) (end 313.96 232.96) (width 0.3048) (layer B.Cu) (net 6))
 (segment (start 339.23 259.5) (end 316.5 259.5) (width 0.3048) (layer B.Cu) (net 12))
 (segment (start 307.27 201.23) (end 308 201.23) (width 0.3048) (layer B.Cu) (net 12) (status C00000))
 (segment (start 304.5 204) (end 307.27 201.23) (width 0.3048) (layer B.Cu) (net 12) (status 800000))
 (segment (start 304.5 252) (end 304.5 204) (width 0.3048) (layer B.Cu) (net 12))
 (segment (start 306 253.5) (end 304.5 252) (width 0.3048) (layer B.Cu) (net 12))
 (segment (start 310.5 253.5) (end 306 253.5) (width 0.3048) (layer B.Cu) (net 12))
 (segment (start 316.5 259.5) (end 310.5 253.5) (width 0.3048) (layer B.Cu) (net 12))
 (segment (start 373.5 187) (end 373.5 248.5) (width 0.3048) (layer B.Cu) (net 12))
 (segment (start 339.23 259.5) (end 337.23 257.5) (width 0.3048) (layer B.Cu) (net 12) (status 800000))
 (segment (start 362.5 259.5) (end 339.23 259.5) (width 0.3048) (layer B.Cu) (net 12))
 (segment (start 373.5 248.5) (end 362.5 259.5) (width 0.3048) (layer B.Cu) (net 12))
 (segment (start 344.27 150.5) (end 344.27 149.23) (width 0.3048) (layer B.Cu) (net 12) (status 400000))
 (segment (start 373.5 187.27) (end 370.5 190.27) (width 0.3048) (layer B.Cu) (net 12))
 (segment (start 373.5 153) (end 373.5 187) (width 0.3048) (layer B.Cu) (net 12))
 (segment (start 373.5 187) (end 373.5 187.27) (width 0.3048) (layer B.Cu) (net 12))
 (segment (start 369 148.5) (end 373.5 153) (width 0.3048) (layer B.Cu) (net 12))
 (segment (start 345 148.5) (end 369 148.5) (width 0.3048) (layer B.Cu) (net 12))
 (segment (start 344.27 149.23) (end 345 148.5) (width 0.3048) (layer B.Cu) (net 12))
 (segment (start 326.84988 232.37694) (end 328.62306 232.37694) (width 0.3048) (layer B.Cu) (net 12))
 (segment (start 341.04 219.96) (end 341.04 184.27) (width 0.3048) (layer B.Cu) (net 12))
 (segment (start 328.62306 232.37694) (end 341.04 219.96) (width 0.3048) (layer B.Cu) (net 12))
 (segment (start 321.15012 233.02718) (end 316.02718 233.02718) (width 0.3048) (layer B.Cu) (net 7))
 (segment (start 309.39 228) (end 309.27 227.88) (width 0.3048) (layer B.Cu) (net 7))
 (segment (start 311 228) (end 309.39 228) (width 0.3048) (layer B.Cu) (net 7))
 (segment (start 316.02718 233.02718) (end 311 228) (width 0.3048) (layer B.Cu) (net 7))
 (segment (start 324 235.5) (end 324 181) (width 0.3048) (layer B.Cu) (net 19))
 (segment (start 324.92354 236.92354) (end 324 236) (width 0.3048) (layer B.Cu) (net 19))
 (segment (start 324 236) (end 324 235.5) (width 0.3048) (layer B.Cu) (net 19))
 (segment (start 326.84988 236.92354) (end 324.92354 236.92354) (width 0.3048) (layer B.Cu) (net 19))
 (segment (start 333.42 179.92) (end 333.42 181.73) (width 0.3048) (layer B.Cu) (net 19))
 (segment (start 332 178.5) (end 333.42 179.92) (width 0.3048) (layer B.Cu) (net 19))
 (segment (start 326.5 178.5) (end 332 178.5) (width 0.3048) (layer B.Cu) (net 19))
 (segment (start 324 181) (end 326.5 178.5) (width 0.3048) (layer B.Cu) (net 19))
 (segment (start 326.84988 235.62306) (end 345.87694 235.62306) (width 0.3048) (layer B.Cu) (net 17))
 (segment (start 335.96 179.04) (end 335.96 181.73) (width 0.3048) (layer B.Cu) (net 17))
 (segment (start 340.251358 174.276025) (end 335.96 179.04) (width 0.3048) (layer B.Cu) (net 17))
 (segment (start 356.39726 174.273972) (end 340.251358 174.276025) (width 0.3048) (layer B.Cu) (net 17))
 (segment (start 362.5 180.5) (end 356.39726 174.273972) (width 0.3048) (layer B.Cu) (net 17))
 (segment (start 362.5 219) (end 362.5 180.5) (width 0.3048) (layer B.Cu) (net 17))
 (segment (start 345.87694 235.62306) (end 362.5 219) (width 0.3048) (layer B.Cu) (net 17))
 (segment (start 321.15012 236.92354) (end 319.57646 236.92354) (width 0.3048) (layer B.Cu) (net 1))
 (segment (start 313.38 243.12) (end 306.73 243.12) (width 0.3048) (layer B.Cu) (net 1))
 (segment (start 319.57646 236.92354) (end 313.38 243.12) (width 0.3048) (layer B.Cu) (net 1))
 (segment (start 326.84988 236.2733) (end 325.7733 236.2733) (width 0.3048) (layer B.Cu) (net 18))
 (segment (start 338.5 191) (end 338.5 184.27) (width 0.3048) (layer B.Cu) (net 18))
 (segment (start 325 204.5) (end 338.5 191) (width 0.3048) (layer B.Cu) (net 18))
 (segment (start 325 235.5) (end 325 204.5) (width 0.3048) (layer B.Cu) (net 18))
 (segment (start 325.7733 236.2733) (end 325 235.5) (width 0.3048) (layer B.Cu) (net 18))
 (segment (start 308 190.23) (end 308 186.08) (width 0.4064) (layer B.Cu) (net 20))
 (segment (start 370.5 178.58) (end 364.02004 178.58) (width 0.4064) (layer B.Cu) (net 21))
 (segment (start 364.02004 178.58) (end 358.96504 173.525) (width 0.4064) (layer B.Cu) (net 21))
 (segment (start 339.91504 154.475) (end 339.91504 160.91504) (width 0.4064) (layer B.Cu) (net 22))
 (segment (start 347.42 168.42) (end 370.5 168.42) (width 0.4064) (layer B.Cu) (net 22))
 (segment (start 339.91504 160.91504) (end 347.42 168.42) (width 0.4064) (layer B.Cu) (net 22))
 (segment (start 336.73496 154.475) (end 336.73496 162.23496) (width 0.4064) (layer B.Cu) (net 25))
 (segment (start 367.73 158.5) (end 364 154.77) (width 0.4064) (layer B.Cu) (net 25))
 (segment (start 368.5 158.5) (end 367.73 158.5) (width 0.4064) (layer B.Cu) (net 25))
 (segment (start 372.5 162.5) (end 368.5 158.5) (width 0.4064) (layer B.Cu) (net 25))
 (segment (start 372.5 170) (end 372.5 162.5) (width 0.4064) (layer B.Cu) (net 25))
 (segment (start 371.5 171) (end 372.5 170) (width 0.4064) (layer B.Cu) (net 25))
 (segment (start 345.5 171) (end 371.5 171) (width 0.4064) (layer B.Cu) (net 25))
 (segment (start 336.73496 162.23496) (end 345.5 171) (width 0.4064) (layer B.Cu) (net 25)))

